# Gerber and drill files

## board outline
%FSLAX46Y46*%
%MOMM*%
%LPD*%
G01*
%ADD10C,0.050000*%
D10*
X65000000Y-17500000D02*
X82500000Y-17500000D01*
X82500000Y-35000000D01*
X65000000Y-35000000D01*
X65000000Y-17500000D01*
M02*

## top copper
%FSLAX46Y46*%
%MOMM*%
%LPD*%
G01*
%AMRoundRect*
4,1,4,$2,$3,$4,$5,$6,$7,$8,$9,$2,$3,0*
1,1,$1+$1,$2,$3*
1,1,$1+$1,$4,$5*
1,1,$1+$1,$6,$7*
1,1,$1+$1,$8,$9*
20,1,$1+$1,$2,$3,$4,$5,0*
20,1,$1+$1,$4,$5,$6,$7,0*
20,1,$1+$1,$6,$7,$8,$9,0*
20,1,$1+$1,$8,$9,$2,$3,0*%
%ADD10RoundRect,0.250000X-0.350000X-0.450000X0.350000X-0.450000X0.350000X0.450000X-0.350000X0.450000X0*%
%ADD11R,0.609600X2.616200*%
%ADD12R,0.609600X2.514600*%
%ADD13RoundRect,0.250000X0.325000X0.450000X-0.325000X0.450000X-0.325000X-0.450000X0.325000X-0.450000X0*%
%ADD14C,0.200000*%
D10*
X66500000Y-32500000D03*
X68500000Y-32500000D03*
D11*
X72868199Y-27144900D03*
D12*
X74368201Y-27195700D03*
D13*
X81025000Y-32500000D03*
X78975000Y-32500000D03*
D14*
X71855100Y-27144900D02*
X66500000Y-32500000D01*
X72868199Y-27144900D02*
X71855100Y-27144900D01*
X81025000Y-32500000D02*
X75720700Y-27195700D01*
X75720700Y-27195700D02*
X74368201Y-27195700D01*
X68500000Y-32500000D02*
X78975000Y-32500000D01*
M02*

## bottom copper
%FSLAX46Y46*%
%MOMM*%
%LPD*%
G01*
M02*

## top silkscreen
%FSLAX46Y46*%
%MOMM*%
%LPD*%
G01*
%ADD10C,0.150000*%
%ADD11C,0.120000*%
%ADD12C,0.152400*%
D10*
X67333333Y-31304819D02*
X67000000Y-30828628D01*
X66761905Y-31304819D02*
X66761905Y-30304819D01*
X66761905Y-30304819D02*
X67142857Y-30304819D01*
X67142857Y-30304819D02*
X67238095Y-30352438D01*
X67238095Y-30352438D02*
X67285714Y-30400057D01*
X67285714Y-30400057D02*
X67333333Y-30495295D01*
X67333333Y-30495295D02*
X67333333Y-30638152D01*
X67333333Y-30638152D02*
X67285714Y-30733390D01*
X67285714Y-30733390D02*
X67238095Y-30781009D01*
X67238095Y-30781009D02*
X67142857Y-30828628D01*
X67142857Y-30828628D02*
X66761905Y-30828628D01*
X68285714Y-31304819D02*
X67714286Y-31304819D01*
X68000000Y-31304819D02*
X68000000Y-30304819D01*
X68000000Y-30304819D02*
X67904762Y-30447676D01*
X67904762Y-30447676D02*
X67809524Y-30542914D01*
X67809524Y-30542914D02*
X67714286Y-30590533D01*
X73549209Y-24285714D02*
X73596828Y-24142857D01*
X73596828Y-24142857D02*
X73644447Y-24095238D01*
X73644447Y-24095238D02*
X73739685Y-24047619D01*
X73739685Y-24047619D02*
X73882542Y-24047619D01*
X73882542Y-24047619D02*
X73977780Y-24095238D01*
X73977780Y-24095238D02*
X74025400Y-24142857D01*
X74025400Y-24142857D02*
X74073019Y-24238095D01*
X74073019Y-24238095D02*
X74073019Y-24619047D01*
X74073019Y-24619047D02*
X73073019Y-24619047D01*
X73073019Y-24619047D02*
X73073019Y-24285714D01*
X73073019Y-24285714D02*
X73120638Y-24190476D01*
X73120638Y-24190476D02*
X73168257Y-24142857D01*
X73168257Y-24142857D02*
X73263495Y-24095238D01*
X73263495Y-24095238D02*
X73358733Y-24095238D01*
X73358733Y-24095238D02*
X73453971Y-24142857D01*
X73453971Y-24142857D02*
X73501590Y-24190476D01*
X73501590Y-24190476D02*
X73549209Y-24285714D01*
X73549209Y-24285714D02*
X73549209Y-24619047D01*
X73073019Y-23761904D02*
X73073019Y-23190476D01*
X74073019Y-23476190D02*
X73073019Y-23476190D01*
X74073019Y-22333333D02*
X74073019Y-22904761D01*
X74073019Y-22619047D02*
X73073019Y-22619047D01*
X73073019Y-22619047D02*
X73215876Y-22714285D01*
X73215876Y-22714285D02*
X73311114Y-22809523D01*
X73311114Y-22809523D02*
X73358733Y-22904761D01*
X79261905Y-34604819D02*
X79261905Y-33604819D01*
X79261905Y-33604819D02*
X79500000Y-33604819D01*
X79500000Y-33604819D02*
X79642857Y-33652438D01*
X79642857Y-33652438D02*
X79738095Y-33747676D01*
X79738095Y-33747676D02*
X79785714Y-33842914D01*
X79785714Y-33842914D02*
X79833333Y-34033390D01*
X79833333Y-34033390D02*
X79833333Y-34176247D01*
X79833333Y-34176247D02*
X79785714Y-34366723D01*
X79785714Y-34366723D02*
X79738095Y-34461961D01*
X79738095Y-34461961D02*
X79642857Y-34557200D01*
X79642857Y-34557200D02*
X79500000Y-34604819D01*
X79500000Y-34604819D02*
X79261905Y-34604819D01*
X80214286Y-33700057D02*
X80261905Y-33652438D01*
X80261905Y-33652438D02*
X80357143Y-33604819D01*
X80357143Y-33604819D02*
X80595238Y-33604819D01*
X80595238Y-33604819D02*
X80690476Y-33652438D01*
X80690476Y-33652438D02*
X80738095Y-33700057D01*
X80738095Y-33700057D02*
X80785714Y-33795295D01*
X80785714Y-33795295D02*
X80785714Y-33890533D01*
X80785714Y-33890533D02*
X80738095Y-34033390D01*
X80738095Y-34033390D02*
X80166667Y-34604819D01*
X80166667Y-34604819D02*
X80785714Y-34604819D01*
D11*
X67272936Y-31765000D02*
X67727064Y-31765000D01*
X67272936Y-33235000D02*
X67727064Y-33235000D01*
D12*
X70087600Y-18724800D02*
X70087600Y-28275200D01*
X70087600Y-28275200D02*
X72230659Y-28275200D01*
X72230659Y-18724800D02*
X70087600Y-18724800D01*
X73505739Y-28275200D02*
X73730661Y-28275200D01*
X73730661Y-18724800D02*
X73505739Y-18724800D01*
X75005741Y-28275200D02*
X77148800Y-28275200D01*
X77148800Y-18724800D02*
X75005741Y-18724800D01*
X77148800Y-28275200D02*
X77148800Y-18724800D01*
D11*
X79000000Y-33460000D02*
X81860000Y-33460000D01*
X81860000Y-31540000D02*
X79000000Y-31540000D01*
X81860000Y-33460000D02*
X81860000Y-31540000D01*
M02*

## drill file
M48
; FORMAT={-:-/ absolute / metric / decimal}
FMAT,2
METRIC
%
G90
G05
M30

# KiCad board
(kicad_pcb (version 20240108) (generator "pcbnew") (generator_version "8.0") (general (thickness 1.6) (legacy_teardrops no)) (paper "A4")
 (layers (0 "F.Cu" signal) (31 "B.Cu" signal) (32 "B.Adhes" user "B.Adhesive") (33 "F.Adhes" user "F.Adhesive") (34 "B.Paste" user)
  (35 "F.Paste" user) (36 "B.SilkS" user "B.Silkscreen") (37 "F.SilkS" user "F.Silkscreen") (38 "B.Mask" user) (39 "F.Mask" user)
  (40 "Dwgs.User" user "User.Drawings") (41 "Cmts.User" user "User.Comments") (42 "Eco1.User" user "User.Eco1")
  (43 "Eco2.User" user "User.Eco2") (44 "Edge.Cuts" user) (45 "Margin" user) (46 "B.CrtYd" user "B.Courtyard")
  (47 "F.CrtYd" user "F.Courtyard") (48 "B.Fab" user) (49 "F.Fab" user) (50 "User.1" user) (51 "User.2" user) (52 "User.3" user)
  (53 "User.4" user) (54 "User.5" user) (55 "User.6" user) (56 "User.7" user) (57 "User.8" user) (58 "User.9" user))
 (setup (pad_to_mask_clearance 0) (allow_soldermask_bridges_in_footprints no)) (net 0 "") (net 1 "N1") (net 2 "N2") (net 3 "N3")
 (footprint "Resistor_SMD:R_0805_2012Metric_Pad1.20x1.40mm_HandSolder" (layer "F.Cu") (at 67.5 32.5)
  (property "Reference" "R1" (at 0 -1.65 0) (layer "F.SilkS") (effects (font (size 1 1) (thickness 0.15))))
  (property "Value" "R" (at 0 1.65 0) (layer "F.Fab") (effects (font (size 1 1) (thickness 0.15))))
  (fp_line (start -0.227064 -0.735) (end 0.227064 -0.735) (stroke (width 0.12) (type solid)) (layer "F.SilkS"))
  (fp_line (start -0.227064 0.735) (end 0.227064 0.735) (stroke (width 0.12) (type solid)) (layer "F.SilkS"))
  (pad "1" smd roundrect (at -1 0) (size 1.2 1.4) (layers "F.Cu" "F.Paste" "F.Mask") (roundrect_rratio 0.208333) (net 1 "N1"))
  (pad "2" smd roundrect (at 1 0) (size 1.2 1.4) (layers "F.Cu" "F.Paste" "F.Mask") (roundrect_rratio 0.208333) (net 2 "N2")))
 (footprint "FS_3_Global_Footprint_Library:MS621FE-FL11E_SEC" (layer "F.Cu") (at 73.6182 23.5 90)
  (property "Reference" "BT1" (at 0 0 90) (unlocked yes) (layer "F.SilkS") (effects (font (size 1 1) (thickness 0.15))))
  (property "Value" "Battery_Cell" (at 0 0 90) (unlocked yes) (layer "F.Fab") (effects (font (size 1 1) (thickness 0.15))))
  (fp_line (start 4.7752 -3.5306) (end -4.7752 -3.5306) (stroke (width 0.1524) (type solid)) (layer "F.SilkS"))
  (fp_line (start -4.7752 -3.5306) (end -4.7752 -1.387541) (stroke (width 0.1524) (type solid)) (layer "F.SilkS"))
  (fp_line (start 4.7752 -1.387541) (end 4.7752 -3.5306) (stroke (width 0.1524) (type solid)) (layer "F.SilkS"))
  (fp_line (start -4.7752 -0.112461) (end -4.7752 0.112461) (stroke (width 0.1524) (type solid)) (layer "F.SilkS"))
  (fp_line (start 4.7752 0.112461) (end 4.7752 -0.112461) (stroke (width 0.1524) (type solid)) (layer "F.SilkS"))
  (fp_line (start -4.7752 1.387541) (end -4.7752 3.5306) (stroke (width 0.1524) (type solid)) (layer "F.SilkS"))
  (fp_line (start 4.7752 3.5306) (end 4.7752 1.387541) (stroke (width 0.1524) (type solid)) (layer "F.SilkS"))
  (fp_line (start -4.7752 3.5306) (end 4.7752 3.5306) (stroke (width 0.1524) (type solid)) (layer "F.SilkS"))
  (pad "1" smd rect (at -3.6449 -0.750001 90) (size 2.6162 0.6096) (layers "F.Cu" "F.Paste" "F.Mask") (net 1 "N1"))
  (pad "2" smd rect (at -3.6957 0.750001 90) (size 2.5146 0.6096) (layers "F.Cu" "F.Paste" "F.Mask") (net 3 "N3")))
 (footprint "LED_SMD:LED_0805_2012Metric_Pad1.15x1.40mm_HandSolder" (layer "F.Cu") (at 80 32.5 180)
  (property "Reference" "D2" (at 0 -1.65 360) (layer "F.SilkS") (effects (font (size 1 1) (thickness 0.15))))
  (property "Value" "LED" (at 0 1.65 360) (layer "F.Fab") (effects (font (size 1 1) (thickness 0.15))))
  (fp_line (start 1 -0.96) (end -1.86 -0.96) (stroke (width 0.12) (type solid)) (layer "F.SilkS"))
  (fp_line (start -1.86 0.96) (end 1 0.96) (stroke (width 0.12) (type solid)) (layer "F.SilkS"))
  (fp_line (start -1.86 -0.96) (end -1.86 0.96) (stroke (width 0.12) (type solid)) (layer "F.SilkS"))
  (pad "1" smd roundrect (at -1.025 0 180) (size 1.15 1.4) (layers "F.Cu" "F.Paste" "F.Mask") (roundrect_rratio 0.217391) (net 3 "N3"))
  (pad "2" smd roundrect (at 1.025 0 180) (size 1.15 1.4) (layers "F.Cu" "F.Paste" "F.Mask") (roundrect_rratio 0.217391) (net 2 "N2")))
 (gr_rect (start 65 17.5) (end 82.5 35) (stroke (width 0.05) (type default)) (fill none) (layer "Edge.Cuts"))
 (segment (start 71.8551 27.1449) (end 66.5 32.5) (width 0.2) (layer "F.Cu") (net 1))
 (segment (start 72.868199 27.1449) (end 71.8551 27.1449) (width 0.2) (layer "F.Cu") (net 1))
 (segment (start 81.025 32.5) (end 75.7207 27.1957) (width 0.2) (layer "F.Cu") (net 3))
 (segment (start 75.7207 27.1957) (end 74.368201 27.1957) (width 0.2) (layer "F.Cu") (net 3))
 (segment (start 68.5 32.5) (end 78.975 32.5) (width 0.2) (layer "F.Cu") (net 2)))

